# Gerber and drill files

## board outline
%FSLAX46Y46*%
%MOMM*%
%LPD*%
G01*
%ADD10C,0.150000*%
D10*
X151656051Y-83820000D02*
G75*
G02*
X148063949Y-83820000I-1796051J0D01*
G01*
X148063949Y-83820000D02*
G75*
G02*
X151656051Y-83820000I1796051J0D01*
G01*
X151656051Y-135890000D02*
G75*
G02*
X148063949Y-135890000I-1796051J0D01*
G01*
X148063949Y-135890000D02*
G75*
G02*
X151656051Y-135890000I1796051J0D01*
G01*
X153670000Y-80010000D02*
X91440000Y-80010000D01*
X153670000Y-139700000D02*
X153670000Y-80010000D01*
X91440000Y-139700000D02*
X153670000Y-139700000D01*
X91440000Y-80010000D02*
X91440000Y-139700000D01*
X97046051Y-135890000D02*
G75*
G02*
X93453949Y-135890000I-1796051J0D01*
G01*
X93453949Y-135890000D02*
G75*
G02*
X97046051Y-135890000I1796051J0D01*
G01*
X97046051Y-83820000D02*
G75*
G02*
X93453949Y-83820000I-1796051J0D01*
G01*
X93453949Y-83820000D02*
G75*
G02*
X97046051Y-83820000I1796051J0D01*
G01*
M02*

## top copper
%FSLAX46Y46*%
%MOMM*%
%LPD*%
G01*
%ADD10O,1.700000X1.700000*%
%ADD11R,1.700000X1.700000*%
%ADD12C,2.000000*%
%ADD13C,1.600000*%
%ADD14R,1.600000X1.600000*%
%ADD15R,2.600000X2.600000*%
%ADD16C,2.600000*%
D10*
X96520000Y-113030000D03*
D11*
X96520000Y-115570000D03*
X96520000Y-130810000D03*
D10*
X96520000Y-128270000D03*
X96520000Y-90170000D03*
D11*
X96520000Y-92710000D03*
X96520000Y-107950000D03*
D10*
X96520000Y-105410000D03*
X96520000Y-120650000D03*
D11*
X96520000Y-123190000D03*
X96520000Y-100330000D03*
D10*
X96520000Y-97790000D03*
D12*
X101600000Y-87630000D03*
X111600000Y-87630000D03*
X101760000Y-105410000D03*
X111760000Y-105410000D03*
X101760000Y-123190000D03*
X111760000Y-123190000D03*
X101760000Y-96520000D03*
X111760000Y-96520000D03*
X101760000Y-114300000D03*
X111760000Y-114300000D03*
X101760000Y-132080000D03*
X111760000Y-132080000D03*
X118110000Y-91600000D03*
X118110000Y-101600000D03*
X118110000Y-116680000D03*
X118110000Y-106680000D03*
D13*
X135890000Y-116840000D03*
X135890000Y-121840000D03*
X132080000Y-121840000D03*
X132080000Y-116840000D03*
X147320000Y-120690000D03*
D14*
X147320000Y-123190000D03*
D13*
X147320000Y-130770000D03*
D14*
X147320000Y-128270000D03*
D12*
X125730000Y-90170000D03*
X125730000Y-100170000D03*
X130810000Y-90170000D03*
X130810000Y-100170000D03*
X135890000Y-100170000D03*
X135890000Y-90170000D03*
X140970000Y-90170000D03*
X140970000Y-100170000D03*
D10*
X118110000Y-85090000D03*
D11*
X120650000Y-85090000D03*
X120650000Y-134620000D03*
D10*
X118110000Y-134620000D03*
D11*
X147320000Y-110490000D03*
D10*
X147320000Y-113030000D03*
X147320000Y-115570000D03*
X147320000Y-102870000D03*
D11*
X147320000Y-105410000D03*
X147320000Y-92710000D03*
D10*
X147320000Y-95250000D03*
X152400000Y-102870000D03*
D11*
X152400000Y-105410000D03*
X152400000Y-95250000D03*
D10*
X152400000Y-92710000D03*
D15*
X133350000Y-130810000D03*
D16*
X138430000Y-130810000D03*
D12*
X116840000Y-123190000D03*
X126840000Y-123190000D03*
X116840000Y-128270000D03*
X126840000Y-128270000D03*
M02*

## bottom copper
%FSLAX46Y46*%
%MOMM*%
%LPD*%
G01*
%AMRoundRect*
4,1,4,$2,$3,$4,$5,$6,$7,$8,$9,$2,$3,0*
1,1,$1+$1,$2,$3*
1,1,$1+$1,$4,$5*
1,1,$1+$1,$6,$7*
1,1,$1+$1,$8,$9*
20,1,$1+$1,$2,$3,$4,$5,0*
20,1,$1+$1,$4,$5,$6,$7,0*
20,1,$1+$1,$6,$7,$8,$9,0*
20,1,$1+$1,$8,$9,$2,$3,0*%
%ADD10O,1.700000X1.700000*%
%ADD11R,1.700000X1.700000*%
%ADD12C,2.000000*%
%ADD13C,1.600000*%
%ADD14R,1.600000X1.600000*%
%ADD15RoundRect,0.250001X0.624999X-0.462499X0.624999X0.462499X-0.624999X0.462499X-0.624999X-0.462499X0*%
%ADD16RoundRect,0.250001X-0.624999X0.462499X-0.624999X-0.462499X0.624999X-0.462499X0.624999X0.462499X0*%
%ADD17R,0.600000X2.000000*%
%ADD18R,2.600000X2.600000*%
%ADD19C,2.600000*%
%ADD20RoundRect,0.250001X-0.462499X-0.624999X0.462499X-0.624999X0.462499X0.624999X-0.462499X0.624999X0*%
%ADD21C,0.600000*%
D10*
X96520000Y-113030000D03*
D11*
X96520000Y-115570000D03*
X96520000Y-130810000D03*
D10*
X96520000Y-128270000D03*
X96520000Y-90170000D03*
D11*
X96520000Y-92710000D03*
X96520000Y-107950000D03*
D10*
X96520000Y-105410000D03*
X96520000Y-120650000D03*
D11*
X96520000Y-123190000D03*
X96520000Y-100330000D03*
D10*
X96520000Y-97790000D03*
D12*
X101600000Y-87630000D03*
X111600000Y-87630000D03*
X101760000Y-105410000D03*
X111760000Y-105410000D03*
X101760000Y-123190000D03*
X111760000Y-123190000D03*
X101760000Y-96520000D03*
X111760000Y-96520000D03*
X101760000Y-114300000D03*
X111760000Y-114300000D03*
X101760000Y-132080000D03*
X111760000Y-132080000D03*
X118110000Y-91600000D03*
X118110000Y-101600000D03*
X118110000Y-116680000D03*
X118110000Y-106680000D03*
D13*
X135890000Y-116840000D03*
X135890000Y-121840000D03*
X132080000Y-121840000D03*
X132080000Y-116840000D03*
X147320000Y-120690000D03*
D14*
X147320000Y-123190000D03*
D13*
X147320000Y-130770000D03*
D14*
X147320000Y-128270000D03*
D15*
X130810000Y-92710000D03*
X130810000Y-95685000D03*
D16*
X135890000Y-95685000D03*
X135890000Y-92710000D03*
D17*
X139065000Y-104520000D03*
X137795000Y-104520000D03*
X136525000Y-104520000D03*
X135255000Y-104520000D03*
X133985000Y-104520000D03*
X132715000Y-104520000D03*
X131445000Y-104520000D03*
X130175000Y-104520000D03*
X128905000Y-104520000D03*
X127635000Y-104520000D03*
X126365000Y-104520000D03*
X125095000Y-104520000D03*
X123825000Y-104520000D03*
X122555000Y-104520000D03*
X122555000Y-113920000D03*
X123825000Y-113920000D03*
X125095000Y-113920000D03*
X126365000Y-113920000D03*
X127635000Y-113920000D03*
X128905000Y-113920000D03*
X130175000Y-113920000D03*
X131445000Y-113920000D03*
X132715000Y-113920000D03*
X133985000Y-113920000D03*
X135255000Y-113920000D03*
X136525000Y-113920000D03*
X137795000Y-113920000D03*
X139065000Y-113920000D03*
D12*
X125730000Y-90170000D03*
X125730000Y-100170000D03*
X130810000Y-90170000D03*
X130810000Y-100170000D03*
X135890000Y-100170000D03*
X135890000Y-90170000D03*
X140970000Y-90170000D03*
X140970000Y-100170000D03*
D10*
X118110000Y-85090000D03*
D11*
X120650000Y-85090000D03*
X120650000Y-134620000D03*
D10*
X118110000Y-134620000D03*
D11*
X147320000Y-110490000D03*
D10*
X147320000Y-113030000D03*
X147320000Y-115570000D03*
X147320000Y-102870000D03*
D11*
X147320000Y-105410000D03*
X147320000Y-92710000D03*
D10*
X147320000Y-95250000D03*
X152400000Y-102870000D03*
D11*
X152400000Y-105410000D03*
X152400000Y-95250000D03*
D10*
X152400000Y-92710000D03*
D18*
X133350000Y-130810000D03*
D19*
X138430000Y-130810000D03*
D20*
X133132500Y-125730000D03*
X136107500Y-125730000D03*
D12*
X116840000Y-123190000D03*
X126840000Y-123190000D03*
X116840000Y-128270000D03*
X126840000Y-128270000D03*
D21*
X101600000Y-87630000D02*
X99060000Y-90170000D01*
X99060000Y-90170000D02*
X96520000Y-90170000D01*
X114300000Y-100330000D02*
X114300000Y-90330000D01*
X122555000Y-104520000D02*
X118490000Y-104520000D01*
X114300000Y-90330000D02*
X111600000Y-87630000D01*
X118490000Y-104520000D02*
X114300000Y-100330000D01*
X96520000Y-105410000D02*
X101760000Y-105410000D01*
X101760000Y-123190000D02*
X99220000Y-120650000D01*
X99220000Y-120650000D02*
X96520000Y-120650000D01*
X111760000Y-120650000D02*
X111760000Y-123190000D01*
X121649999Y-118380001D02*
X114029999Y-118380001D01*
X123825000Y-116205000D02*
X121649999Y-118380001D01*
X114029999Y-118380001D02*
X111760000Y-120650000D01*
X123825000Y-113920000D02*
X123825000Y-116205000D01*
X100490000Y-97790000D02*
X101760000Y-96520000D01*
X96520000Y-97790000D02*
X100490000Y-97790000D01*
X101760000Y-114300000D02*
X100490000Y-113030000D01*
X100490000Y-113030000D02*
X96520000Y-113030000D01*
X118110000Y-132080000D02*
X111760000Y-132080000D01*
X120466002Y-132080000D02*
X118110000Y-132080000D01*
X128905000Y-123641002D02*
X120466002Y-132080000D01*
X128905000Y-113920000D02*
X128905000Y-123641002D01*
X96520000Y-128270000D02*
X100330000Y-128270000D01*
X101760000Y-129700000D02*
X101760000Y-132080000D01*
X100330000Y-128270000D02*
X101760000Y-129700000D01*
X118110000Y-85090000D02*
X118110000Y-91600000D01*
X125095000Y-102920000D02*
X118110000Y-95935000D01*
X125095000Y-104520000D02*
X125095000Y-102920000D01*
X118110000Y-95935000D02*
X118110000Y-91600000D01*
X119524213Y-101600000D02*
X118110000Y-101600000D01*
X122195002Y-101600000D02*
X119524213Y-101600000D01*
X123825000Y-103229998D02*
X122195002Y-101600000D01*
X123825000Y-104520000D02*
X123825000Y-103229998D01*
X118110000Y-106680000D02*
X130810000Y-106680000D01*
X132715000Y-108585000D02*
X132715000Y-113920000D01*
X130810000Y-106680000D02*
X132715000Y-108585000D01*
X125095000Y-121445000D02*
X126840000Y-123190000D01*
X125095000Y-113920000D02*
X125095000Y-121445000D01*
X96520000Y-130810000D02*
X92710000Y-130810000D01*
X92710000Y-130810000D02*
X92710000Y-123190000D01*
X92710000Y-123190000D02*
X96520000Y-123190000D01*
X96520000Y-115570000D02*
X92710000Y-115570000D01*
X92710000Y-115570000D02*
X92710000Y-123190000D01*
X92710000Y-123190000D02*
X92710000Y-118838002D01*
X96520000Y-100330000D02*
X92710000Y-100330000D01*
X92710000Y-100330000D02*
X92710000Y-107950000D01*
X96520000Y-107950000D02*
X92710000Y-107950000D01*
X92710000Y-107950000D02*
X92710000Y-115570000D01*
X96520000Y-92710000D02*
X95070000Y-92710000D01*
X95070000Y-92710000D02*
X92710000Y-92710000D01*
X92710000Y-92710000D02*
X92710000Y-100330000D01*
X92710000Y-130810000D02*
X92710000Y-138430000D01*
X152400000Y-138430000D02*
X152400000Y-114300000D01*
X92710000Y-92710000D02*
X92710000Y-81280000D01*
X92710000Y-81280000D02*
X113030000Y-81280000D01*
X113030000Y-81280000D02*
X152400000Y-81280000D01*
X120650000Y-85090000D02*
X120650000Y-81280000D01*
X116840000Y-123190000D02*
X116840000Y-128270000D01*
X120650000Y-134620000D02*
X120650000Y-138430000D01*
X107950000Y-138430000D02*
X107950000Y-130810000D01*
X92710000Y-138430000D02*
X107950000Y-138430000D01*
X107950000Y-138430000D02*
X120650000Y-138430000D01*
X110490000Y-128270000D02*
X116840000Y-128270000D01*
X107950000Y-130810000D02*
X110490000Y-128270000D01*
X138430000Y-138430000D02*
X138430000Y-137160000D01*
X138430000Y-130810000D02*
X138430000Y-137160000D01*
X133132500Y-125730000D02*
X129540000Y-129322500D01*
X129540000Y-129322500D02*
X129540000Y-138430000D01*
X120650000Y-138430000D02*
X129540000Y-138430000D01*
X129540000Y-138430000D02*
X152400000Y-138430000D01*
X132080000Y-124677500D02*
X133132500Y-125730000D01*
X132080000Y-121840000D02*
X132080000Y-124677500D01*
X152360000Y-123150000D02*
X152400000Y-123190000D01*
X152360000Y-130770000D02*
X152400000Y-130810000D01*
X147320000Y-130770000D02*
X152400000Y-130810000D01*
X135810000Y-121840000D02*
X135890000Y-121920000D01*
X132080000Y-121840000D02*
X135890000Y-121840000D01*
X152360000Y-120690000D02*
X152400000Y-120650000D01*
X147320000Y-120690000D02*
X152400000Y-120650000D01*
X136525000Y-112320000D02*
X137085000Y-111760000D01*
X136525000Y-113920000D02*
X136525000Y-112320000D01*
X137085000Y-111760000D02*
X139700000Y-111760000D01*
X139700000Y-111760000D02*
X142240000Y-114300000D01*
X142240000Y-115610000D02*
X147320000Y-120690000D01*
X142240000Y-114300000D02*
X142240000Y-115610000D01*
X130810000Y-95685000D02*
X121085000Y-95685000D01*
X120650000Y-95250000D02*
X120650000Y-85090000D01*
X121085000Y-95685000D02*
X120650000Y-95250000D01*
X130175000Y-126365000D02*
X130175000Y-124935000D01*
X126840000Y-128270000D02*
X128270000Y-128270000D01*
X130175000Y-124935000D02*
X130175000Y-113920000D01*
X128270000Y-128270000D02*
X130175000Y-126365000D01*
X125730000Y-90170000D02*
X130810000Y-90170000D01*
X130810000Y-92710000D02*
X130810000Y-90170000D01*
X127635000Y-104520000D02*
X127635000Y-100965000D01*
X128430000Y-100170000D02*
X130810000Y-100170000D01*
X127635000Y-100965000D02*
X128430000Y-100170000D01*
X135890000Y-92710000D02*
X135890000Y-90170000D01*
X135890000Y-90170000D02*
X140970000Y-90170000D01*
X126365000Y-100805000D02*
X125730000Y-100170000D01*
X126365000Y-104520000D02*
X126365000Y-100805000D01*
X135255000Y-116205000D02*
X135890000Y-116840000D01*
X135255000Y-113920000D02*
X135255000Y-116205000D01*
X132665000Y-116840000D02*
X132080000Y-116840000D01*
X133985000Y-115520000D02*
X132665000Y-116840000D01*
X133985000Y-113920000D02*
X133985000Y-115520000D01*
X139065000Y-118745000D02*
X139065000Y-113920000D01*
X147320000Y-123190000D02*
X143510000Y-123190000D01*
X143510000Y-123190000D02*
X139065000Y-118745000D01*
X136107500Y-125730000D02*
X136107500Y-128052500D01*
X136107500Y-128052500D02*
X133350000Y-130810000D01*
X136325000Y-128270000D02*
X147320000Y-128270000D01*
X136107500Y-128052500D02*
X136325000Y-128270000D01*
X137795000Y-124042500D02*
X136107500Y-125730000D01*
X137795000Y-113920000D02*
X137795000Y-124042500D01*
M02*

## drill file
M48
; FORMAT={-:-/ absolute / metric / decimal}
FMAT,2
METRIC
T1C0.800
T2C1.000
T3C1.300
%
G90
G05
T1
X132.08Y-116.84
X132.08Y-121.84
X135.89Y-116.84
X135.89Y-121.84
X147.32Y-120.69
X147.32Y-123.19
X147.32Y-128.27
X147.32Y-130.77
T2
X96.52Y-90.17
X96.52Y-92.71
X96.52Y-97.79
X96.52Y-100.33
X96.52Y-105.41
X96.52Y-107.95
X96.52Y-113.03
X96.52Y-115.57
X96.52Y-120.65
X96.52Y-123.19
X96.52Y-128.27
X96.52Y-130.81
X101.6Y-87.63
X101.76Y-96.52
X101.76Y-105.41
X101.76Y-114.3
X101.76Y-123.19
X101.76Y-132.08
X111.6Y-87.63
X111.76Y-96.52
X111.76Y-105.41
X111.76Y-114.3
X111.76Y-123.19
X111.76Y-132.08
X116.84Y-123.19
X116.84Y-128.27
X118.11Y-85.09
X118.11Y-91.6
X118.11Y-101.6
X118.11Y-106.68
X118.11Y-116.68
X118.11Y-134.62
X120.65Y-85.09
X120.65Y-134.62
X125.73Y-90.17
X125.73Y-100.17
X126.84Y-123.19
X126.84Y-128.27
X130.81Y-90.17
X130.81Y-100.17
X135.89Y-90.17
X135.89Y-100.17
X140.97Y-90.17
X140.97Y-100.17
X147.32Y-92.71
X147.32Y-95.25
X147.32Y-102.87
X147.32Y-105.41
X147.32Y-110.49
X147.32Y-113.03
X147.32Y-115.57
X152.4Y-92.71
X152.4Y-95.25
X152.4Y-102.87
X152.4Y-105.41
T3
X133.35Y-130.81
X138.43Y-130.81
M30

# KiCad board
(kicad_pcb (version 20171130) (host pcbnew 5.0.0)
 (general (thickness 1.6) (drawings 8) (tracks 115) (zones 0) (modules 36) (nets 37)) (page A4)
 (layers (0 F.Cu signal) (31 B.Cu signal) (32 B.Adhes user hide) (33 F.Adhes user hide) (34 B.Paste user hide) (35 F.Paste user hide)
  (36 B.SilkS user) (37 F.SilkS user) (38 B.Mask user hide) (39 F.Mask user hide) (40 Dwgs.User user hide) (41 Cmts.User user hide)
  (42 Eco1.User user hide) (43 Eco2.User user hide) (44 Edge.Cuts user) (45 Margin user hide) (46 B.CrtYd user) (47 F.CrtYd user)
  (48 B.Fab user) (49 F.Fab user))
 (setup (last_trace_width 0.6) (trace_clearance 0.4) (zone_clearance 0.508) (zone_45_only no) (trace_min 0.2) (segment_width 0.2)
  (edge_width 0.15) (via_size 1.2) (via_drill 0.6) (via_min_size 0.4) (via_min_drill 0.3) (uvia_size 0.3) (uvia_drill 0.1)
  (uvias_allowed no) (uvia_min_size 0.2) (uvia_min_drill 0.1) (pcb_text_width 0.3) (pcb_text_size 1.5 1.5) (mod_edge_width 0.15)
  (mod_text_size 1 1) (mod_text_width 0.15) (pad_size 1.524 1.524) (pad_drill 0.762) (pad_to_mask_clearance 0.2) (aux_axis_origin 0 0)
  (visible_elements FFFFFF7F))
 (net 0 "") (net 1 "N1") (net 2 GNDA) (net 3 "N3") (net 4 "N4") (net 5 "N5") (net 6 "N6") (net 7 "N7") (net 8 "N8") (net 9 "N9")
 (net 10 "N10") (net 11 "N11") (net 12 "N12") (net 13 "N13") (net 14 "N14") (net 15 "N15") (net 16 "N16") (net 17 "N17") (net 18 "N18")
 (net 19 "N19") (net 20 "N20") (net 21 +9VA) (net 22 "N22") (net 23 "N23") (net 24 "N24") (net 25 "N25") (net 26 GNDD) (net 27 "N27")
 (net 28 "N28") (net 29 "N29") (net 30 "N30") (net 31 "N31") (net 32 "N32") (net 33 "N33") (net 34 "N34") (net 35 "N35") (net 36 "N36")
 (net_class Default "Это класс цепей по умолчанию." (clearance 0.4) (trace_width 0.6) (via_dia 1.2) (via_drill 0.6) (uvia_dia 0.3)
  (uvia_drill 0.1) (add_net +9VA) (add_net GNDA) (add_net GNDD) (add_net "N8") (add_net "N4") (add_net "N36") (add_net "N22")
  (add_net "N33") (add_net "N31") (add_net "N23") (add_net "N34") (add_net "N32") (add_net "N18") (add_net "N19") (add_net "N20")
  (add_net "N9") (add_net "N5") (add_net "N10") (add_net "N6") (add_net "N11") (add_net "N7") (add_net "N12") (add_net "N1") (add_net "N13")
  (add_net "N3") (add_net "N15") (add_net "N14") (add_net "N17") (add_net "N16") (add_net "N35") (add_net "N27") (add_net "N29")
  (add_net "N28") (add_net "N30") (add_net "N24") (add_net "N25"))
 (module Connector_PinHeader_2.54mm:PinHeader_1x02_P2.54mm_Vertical (layer F.Cu) (at 96.52 115.57 180)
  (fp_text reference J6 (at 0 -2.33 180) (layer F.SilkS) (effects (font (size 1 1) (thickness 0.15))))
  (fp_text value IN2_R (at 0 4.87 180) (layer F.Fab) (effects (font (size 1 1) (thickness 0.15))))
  (pad 2 thru_hole oval (at 0 2.54 180) (size 1.7 1.7) (drill 1) (layers *.Cu *.Mask) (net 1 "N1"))
  (pad 1 thru_hole rect (at 0 0 180) (size 1.7 1.7) (drill 1) (layers *.Cu *.Mask) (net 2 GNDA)))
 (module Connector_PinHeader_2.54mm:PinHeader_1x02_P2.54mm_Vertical (layer F.Cu) (at 96.52 130.81 180)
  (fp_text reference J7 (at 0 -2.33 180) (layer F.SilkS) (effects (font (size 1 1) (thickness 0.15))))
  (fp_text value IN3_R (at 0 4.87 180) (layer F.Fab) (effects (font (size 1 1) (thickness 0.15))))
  (pad 1 thru_hole rect (at 0 0 180) (size 1.7 1.7) (drill 1) (layers *.Cu *.Mask) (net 2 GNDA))
  (pad 2 thru_hole oval (at 0 2.54 180) (size 1.7 1.7) (drill 1) (layers *.Cu *.Mask) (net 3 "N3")))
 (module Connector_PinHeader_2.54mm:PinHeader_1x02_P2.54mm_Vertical (layer F.Cu) (at 96.52 92.71 180)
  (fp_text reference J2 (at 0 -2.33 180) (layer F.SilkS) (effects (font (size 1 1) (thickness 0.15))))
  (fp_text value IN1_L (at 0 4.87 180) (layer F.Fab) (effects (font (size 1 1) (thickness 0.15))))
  (pad 2 thru_hole oval (at 0 2.54 180) (size 1.7 1.7) (drill 1) (layers *.Cu *.Mask) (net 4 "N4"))
  (pad 1 thru_hole rect (at 0 0 180) (size 1.7 1.7) (drill 1) (layers *.Cu *.Mask) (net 2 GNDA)))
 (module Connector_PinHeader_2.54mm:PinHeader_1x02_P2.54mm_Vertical (layer F.Cu) (at 96.52 107.95 180)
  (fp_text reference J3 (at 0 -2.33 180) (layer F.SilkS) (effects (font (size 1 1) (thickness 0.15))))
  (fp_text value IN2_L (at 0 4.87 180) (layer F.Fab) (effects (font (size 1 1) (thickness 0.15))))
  (pad 1 thru_hole rect (at 0 0 180) (size 1.7 1.7) (drill 1) (layers *.Cu *.Mask) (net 2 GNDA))
  (pad 2 thru_hole oval (at 0 2.54 180) (size 1.7 1.7) (drill 1) (layers *.Cu *.Mask) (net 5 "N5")))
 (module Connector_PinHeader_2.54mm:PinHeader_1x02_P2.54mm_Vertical (layer F.Cu) (at 96.52 123.19 180)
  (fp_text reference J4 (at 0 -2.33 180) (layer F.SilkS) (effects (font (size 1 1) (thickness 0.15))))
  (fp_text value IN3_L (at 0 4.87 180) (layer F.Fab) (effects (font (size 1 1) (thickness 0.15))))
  (pad 2 thru_hole oval (at 0 2.54 180) (size 1.7 1.7) (drill 1) (layers *.Cu *.Mask) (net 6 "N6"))
  (pad 1 thru_hole rect (at 0 0 180) (size 1.7 1.7) (drill 1) (layers *.Cu *.Mask) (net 2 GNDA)))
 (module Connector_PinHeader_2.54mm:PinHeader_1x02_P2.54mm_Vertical (layer F.Cu) (at 96.52 100.33 180)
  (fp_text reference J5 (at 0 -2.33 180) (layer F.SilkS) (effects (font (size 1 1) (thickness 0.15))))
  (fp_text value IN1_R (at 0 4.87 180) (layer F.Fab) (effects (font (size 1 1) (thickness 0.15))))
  (pad 1 thru_hole rect (at 0 0 180) (size 1.7 1.7) (drill 1) (layers *.Cu *.Mask) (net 2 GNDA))
  (pad 2 thru_hole oval (at 0 2.54 180) (size 1.7 1.7) (drill 1) (layers *.Cu *.Mask) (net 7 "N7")))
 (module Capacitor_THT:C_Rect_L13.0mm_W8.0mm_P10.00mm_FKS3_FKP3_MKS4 (layer F.Cu) (at 111.6 87.63 180)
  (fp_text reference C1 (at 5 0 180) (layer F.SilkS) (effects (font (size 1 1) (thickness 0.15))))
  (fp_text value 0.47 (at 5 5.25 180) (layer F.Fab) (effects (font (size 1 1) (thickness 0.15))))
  (pad 2 thru_hole circle (at 10 0 180) (size 2 2) (drill 1) (layers *.Cu *.Mask) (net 4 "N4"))
  (pad 1 thru_hole circle (at 0 0 180) (size 2 2) (drill 1) (layers *.Cu *.Mask) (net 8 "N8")))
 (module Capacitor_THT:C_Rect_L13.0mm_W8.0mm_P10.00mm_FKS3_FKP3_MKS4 (layer F.Cu) (at 111.76 105.41 180)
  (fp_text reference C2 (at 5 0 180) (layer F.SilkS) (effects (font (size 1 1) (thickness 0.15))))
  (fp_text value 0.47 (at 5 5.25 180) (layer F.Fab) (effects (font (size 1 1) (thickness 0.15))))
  (pad 2 thru_hole circle (at 10 0 180) (size 2 2) (drill 1) (layers *.Cu *.Mask) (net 5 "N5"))
  (pad 1 thru_hole circle (at 0 0 180) (size 2 2) (drill 1) (layers *.Cu *.Mask) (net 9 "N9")))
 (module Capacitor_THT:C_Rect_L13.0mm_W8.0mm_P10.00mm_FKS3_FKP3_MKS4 (layer F.Cu) (at 111.76 123.19 180)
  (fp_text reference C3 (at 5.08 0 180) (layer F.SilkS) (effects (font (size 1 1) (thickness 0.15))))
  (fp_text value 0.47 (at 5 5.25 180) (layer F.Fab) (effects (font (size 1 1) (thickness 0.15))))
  (pad 2 thru_hole circle (at 10 0 180) (size 2 2) (drill 1) (layers *.Cu *.Mask) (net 6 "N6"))
  (pad 1 thru_hole circle (at 0 0 180) (size 2 2) (drill 1) (layers *.Cu *.Mask) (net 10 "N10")))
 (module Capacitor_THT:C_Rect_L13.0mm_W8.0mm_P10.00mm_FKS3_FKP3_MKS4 (layer F.Cu) (at 111.76 96.52 180)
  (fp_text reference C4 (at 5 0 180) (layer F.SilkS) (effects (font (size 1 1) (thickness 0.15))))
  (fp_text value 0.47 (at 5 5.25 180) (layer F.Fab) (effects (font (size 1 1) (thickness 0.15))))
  (pad 2 thru_hole circle (at 10 0 180) (size 2 2) (drill 1) (layers *.Cu *.Mask) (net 7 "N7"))
  (pad 1 thru_hole circle (at 0 0 180) (size 2 2) (drill 1) (layers *.Cu *.Mask) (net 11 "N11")))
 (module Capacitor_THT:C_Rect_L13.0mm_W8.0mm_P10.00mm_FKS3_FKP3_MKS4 (layer F.Cu) (at 111.76 114.3 180)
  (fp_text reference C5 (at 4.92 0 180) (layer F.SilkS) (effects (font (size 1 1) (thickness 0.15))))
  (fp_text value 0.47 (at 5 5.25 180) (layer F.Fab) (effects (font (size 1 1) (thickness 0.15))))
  (pad 2 thru_hole circle (at 10 0 180) (size 2 2) (drill 1) (layers *.Cu *.Mask) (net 1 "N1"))
  (pad 1 thru_hole circle (at 0 0 180) (size 2 2) (drill 1) (layers *.Cu *.Mask) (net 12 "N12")))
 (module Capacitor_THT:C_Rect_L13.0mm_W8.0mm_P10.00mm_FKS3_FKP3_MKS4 (layer F.Cu) (at 111.76 132.08 180)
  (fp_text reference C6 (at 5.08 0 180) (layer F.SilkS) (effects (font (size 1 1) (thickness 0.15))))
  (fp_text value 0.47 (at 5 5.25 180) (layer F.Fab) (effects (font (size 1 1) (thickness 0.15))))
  (pad 2 thru_hole circle (at 10 0 180) (size 2 2) (drill 1) (layers *.Cu *.Mask) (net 3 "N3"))
  (pad 1 thru_hole circle (at 0 0 180) (size 2 2) (drill 1) (layers *.Cu *.Mask) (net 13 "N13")))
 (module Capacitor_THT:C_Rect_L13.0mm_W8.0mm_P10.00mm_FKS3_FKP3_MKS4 (layer F.Cu) (at 118.11 101.6 90)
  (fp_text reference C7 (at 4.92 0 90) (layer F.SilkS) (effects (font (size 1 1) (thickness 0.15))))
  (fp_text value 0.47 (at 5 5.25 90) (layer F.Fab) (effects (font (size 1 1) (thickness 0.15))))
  (pad 2 thru_hole circle (at 10 0 90) (size 2 2) (drill 1) (layers *.Cu *.Mask) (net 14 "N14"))
  (pad 1 thru_hole circle (at 0 0 90) (size 2 2) (drill 1) (layers *.Cu *.Mask) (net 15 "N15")))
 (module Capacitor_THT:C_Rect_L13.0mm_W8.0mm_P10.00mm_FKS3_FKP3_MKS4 (layer F.Cu) (at 118.11 106.68 270)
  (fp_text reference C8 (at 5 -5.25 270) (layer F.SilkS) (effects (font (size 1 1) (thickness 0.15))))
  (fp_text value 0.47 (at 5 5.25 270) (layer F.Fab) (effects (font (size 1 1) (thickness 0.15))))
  (pad 2 thru_hole circle (at 10 0 270) (size 2 2) (drill 1) (layers *.Cu *.Mask) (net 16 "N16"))
  (pad 1 thru_hole circle (at 0 0 270) (size 2 2) (drill 1) (layers *.Cu *.Mask) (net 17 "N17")))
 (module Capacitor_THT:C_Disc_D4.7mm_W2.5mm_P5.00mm (layer F.Cu) (at 135.89 121.84 90)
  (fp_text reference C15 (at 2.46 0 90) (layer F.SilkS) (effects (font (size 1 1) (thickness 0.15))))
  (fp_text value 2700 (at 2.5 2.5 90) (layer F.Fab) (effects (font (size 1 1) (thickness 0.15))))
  (pad 2 thru_hole circle (at 5 0 90) (size 1.6 1.6) (drill 0.8) (layers *.Cu *.Mask) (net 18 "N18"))
  (pad 1 thru_hole circle (at 0 0 90) (size 1.6 1.6) (drill 0.8) (layers *.Cu *.Mask) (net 2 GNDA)))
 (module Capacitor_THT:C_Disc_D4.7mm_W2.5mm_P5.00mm (layer F.Cu) (at 132.08 116.84 270)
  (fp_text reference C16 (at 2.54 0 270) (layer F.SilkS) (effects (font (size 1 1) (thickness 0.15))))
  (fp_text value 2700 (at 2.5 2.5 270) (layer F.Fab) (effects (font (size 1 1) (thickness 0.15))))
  (pad 2 thru_hole circle (at 5 0 270) (size 1.6 1.6) (drill 0.8) (layers *.Cu *.Mask) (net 2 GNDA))
  (pad 1 thru_hole circle (at 0 0 270) (size 1.6 1.6) (drill 0.8) (layers *.Cu *.Mask) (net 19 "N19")))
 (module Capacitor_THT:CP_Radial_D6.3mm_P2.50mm (layer F.Cu) (at 147.32 123.19 90)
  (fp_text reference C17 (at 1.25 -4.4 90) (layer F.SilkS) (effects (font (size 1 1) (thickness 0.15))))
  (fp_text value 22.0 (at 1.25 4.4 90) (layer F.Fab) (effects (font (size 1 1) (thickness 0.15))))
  (pad 2 thru_hole circle (at 2.5 0 90) (size 1.6 1.6) (drill 0.8) (layers *.Cu *.Mask) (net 2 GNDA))
  (pad 1 thru_hole rect (at 0 0 90) (size 1.6 1.6) (drill 0.8) (layers *.Cu *.Mask) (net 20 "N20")))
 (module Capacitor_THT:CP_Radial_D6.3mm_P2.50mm (layer F.Cu) (at 147.32 128.27 270)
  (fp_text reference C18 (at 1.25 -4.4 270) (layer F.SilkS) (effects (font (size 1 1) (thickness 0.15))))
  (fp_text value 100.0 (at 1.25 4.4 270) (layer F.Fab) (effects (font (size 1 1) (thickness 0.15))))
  (pad 2 thru_hole circle (at 2.5 0 270) (size 1.6 1.6) (drill 0.8) (layers *.Cu *.Mask) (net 2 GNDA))
  (pad 1 thru_hole rect (at 0 0 270) (size 1.6 1.6) (drill 0.8) (layers *.Cu *.Mask) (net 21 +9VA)))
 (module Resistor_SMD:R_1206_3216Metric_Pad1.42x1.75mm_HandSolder (layer B.Cu) (at 130.81 94.1975 90)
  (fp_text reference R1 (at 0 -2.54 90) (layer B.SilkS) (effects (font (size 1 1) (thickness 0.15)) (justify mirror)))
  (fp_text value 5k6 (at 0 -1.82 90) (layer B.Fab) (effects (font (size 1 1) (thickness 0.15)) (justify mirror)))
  (pad 2 smd roundrect (at 1.4875 0 90) (size 1.425 1.75) (layers B.Cu B.Paste B.Mask) (roundrect_rratio 0.175439) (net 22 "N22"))
  (pad 1 smd roundrect (at -1.4875 0 90) (size 1.425 1.75) (layers B.Cu B.Paste B.Mask) (roundrect_rratio 0.175439) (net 2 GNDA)))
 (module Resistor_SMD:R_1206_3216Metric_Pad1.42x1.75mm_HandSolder (layer B.Cu) (at 135.89 94.1975 270)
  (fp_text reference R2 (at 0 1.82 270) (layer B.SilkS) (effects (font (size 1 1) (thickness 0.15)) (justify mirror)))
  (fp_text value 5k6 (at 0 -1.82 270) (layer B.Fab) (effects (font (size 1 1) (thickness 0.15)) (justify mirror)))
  (pad 2 smd roundrect (at 1.4875 0 270) (size 1.425 1.75) (layers B.Cu B.Paste B.Mask) (roundrect_rratio 0.175439) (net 2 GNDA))
  (pad 1 smd roundrect (at -1.4875 0 270) (size 1.425 1.75) (layers B.Cu B.Paste B.Mask) (roundrect_rratio 0.175439) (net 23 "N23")))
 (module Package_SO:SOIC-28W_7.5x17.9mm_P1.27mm (layer B.Cu) (at 130.81 109.22 90)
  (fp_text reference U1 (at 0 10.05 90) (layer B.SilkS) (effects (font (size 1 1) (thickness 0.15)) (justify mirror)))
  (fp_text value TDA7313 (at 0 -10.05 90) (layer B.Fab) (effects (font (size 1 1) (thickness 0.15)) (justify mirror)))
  (pad 28 smd rect (at 4.7 8.255 90) (size 2 0.6) (layers B.Cu B.Paste B.Mask) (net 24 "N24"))
  (pad 27 smd rect (at 4.7 6.985 90) (size 2 0.6) (layers B.Cu B.Paste B.Mask) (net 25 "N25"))
  (pad 26 smd rect (at 4.7 5.715 90) (size 2 0.6) (layers B.Cu B.Paste B.Mask) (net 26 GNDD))
  (pad 25 smd rect (at 4.7 4.445 90) (size 2 0.6) (layers B.Cu B.Paste B.Mask) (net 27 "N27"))
  (pad 24 smd rect (at 4.7 3.175 90) (size 2 0.6) (layers B.Cu B.Paste B.Mask) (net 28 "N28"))
  (pad 23 smd rect (at 4.7 1.905 90) (size 2 0.6) (layers B.Cu B.Paste B.Mask) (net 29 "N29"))
  (pad 22 smd rect (at 4.7 0.635 90) (size 2 0.6) (layers B.Cu B.Paste B.Mask) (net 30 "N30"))
  (pad 21 smd rect (at 4.7 -0.635 90) (size 2 0.6) (layers B.Cu B.Paste B.Mask) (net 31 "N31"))
  (pad 20 smd rect (at 4.7 -1.905 90) (size 2 0.6) (layers B.Cu B.Paste B.Mask) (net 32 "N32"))
  (pad 19 smd rect (at 4.7 -3.175 90) (size 2 0.6) (layers B.Cu B.Paste B.Mask) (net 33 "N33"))
  (pad 18 smd rect (at 4.7 -4.445 90) (size 2 0.6) (layers B.Cu B.Paste B.Mask) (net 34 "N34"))
  (pad 17 smd rect (at 4.7 -5.715 90) (size 2 0.6) (layers B.Cu B.Paste B.Mask) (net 14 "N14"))
  (pad 16 smd rect (at 4.7 -6.985 90) (size 2 0.6) (layers B.Cu B.Paste B.Mask) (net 15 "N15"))
  (pad 15 smd rect (at 4.7 -8.255 90) (size 2 0.6) (layers B.Cu B.Paste B.Mask) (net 8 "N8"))
  (pad 14 smd rect (at -4.7 -8.255 90) (size 2 0.6) (layers B.Cu B.Paste B.Mask) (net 9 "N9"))
  (pad 13 smd rect (at -4.7 -6.985 90) (size 2 0.6) (layers B.Cu B.Paste B.Mask) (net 10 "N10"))
  (pad 12 smd rect (at -4.7 -5.715 90) (size 2 0.6) (layers B.Cu B.Paste B.Mask) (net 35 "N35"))
  (pad 11 smd rect (at -4.7 -4.445 90) (size 2 0.6) (layers B.Cu B.Paste B.Mask) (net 11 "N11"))
  (pad 10 smd rect (at -4.7 -3.175 90) (size 2 0.6) (layers B.Cu B.Paste B.Mask) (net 12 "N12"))
  (pad 9 smd rect (at -4.7 -1.905 90) (size 2 0.6) (layers B.Cu B.Paste B.Mask) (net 13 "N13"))
  (pad 8 smd rect (at -4.7 -0.635 90) (size 2 0.6) (layers B.Cu B.Paste B.Mask) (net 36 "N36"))
  (pad 7 smd rect (at -4.7 0.635 90) (size 2 0.6) (layers B.Cu B.Paste B.Mask) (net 16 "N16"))
  (pad 6 smd rect (at -4.7 1.905 90) (size 2 0.6) (layers B.Cu B.Paste B.Mask) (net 17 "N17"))
  (pad 5 smd rect (at -4.7 3.175 90) (size 2 0.6) (layers B.Cu B.Paste B.Mask) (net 19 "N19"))
  (pad 4 smd rect (at -4.7 4.445 90) (size 2 0.6) (layers B.Cu B.Paste B.Mask) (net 18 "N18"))
  (pad 3 smd rect (at -4.7 5.715 90) (size 2 0.6) (layers B.Cu B.Paste B.Mask) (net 2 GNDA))
  (pad 2 smd rect (at -4.7 6.985 90) (size 2 0.6) (layers B.Cu B.Paste B.Mask) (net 21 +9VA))
  (pad 1 smd rect (at -4.7 8.255 90) (size 2 0.6) (layers B.Cu B.Paste B.Mask) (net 20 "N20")))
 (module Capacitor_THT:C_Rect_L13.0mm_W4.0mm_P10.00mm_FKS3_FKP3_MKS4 (layer F.Cu) (at 125.73 90.17 270)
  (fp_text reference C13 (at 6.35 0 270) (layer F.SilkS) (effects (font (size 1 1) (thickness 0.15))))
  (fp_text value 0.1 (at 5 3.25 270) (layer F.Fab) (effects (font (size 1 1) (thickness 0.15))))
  (pad 1 thru_hole circle (at 0 0 270) (size 2 2) (drill 1) (layers *.Cu *.Mask) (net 22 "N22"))
  (pad 2 thru_hole circle (at 10 0 270) (size 2 2) (drill 1) (layers *.Cu *.Mask) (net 34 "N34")))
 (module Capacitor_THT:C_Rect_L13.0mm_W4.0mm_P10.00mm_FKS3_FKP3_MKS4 (layer F.Cu) (at 130.81 90.17 270)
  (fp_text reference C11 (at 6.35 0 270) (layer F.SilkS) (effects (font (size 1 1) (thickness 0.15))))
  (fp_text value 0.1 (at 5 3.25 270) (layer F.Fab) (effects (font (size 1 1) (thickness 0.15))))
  (pad 1 thru_hole circle (at 0 0 270) (size 2 2) (drill 1) (layers *.Cu *.Mask) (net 22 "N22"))
  (pad 2 thru_hole circle (at 10 0 270) (size 2 2) (drill 1) (layers *.Cu *.Mask) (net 33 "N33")))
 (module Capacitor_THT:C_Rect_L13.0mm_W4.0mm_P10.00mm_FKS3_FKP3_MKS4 (layer F.Cu) (at 135.89 100.17 90)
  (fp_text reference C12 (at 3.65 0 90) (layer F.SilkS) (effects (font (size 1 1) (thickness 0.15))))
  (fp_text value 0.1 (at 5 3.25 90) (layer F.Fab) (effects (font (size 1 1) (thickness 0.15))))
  (pad 1 thru_hole circle (at 0 0 90) (size 2 2) (drill 1) (layers *.Cu *.Mask) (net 31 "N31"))
  (pad 2 thru_hole circle (at 10 0 90) (size 2 2) (drill 1) (layers *.Cu *.Mask) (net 23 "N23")))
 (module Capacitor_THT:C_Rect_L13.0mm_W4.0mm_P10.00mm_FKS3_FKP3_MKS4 (layer F.Cu) (at 140.97 100.17 90)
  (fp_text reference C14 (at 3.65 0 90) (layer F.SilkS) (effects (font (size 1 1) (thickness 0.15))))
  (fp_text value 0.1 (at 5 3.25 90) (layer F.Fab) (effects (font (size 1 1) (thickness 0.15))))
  (pad 2 thru_hole circle (at 10 0 90) (size 2 2) (drill 1) (layers *.Cu *.Mask) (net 23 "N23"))
  (pad 1 thru_hole circle (at 0 0 90) (size 2 2) (drill 1) (layers *.Cu *.Mask) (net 32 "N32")))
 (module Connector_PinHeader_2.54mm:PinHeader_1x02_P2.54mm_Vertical (layer F.Cu) (at 120.65 85.09 270)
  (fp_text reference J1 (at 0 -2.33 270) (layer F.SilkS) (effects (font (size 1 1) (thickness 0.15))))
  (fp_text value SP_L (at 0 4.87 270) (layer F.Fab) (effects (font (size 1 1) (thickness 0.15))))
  (pad 2 thru_hole oval (at 0 2.54 270) (size 1.7 1.7) (drill 1) (layers *.Cu *.Mask) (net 14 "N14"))
  (pad 1 thru_hole rect (at 0 0 270) (size 1.7 1.7) (drill 1) (layers *.Cu *.Mask) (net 2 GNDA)))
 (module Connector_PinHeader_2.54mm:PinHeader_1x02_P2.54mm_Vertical (layer F.Cu) (at 120.65 134.62 270)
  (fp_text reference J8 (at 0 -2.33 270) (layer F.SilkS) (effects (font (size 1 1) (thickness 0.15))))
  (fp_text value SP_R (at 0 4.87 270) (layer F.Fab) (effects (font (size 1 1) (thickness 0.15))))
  (pad 1 thru_hole rect (at 0 0 270) (size 1.7 1.7) (drill 1) (layers *.Cu *.Mask) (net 2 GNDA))
  (pad 2 thru_hole oval (at 0 2.54 270) (size 1.7 1.7) (drill 1) (layers *.Cu *.Mask) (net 16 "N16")))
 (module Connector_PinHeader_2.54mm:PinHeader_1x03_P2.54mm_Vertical (layer F.Cu) (at 147.32 110.49)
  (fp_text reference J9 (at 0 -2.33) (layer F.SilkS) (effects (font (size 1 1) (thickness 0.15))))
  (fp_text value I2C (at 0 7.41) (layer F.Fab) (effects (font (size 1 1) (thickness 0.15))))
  (pad 1 thru_hole rect (at 0 0) (size 1.7 1.7) (drill 1) (layers *.Cu *.Mask) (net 24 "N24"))
  (pad 2 thru_hole oval (at 0 2.54) (size 1.7 1.7) (drill 1) (layers *.Cu *.Mask) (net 25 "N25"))
  (pad 3 thru_hole oval (at 0 5.08) (size 1.7 1.7) (drill 1) (layers *.Cu *.Mask) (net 26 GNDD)))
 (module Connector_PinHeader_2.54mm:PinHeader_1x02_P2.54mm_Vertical (layer F.Cu) (at 147.32 105.41 180)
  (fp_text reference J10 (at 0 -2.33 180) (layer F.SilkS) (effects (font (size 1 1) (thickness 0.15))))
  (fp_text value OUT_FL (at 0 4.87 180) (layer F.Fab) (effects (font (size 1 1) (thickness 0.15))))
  (pad 2 thru_hole oval (at 0 2.54 180) (size 1.7 1.7) (drill 1) (layers *.Cu *.Mask) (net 27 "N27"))
  (pad 1 thru_hole rect (at 0 0 180) (size 1.7 1.7) (drill 1) (layers *.Cu *.Mask) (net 2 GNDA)))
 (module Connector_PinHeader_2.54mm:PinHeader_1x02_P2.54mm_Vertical (layer F.Cu) (at 147.32 92.71)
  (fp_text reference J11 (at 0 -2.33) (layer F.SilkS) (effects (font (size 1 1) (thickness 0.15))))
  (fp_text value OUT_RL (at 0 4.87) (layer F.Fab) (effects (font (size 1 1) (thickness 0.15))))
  (pad 1 thru_hole rect (at 0 0) (size 1.7 1.7) (drill 1) (layers *.Cu *.Mask) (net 2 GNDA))
  (pad 2 thru_hole oval (at 0 2.54) (size 1.7 1.7) (drill 1) (layers *.Cu *.Mask) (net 29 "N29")))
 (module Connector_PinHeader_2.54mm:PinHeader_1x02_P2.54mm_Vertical (layer F.Cu) (at 152.4 105.41 180)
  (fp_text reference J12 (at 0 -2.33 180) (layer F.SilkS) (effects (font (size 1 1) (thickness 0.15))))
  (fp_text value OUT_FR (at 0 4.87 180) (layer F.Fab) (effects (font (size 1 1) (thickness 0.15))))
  (pad 2 thru_hole oval (at 0 2.54 180) (size 1.7 1.7) (drill 1) (layers *.Cu *.Mask) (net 28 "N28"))
  (pad 1 thru_hole rect (at 0 0 180) (size 1.7 1.7) (drill 1) (layers *.Cu *.Mask) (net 2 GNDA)))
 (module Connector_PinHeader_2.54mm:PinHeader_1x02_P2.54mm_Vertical (layer F.Cu) (at 152.4 95.25 180)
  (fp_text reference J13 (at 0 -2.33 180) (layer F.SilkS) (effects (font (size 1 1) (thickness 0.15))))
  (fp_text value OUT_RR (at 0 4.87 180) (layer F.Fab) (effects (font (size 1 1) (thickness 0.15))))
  (pad 1 thru_hole rect (at 0 0 180) (size 1.7 1.7) (drill 1) (layers *.Cu *.Mask) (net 2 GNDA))
  (pad 2 thru_hole oval (at 0 2.54 180) (size 1.7 1.7) (drill 1) (layers *.Cu *.Mask) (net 30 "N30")))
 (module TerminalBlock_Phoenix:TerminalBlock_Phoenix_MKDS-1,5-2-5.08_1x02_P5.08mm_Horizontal (layer F.Cu) (at 133.35 130.81)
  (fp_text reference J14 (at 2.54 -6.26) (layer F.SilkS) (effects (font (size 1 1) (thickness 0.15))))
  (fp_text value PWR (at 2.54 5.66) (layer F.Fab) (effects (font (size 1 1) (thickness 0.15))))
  (pad 1 thru_hole rect (at 0 0) (size 2.6 2.6) (drill 1.3) (layers *.Cu *.Mask) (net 21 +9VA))
  (pad 2 thru_hole circle (at 5.08 0) (size 2.6 2.6) (drill 1.3) (layers *.Cu *.Mask) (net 2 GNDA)))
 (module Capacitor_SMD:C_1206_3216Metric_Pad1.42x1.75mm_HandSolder (layer B.Cu) (at 134.62 125.73)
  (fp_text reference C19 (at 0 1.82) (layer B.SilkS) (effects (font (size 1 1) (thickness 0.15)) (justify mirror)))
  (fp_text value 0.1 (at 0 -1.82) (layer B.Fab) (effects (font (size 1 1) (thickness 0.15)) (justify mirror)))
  (pad 1 smd roundrect (at -1.4875 0) (size 1.425 1.75) (layers B.Cu B.Paste B.Mask) (roundrect_rratio 0.175439) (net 2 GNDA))
  (pad 2 smd roundrect (at 1.4875 0) (size 1.425 1.75) (layers B.Cu B.Paste B.Mask) (roundrect_rratio 0.175439) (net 21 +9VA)))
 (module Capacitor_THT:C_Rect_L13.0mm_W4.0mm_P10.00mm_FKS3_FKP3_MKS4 (layer F.Cu) (at 116.84 123.19)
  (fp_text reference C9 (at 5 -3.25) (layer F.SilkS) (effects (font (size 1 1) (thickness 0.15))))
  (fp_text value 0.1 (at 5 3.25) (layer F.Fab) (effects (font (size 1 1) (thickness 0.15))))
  (pad 1 thru_hole circle (at 0 0) (size 2 2) (drill 1) (layers *.Cu *.Mask) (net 2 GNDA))
  (pad 2 thru_hole circle (at 10 0) (size 2 2) (drill 1) (layers *.Cu *.Mask) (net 35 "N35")))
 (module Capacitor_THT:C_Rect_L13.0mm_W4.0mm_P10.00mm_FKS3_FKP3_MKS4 (layer F.Cu) (at 126.84 128.27 180)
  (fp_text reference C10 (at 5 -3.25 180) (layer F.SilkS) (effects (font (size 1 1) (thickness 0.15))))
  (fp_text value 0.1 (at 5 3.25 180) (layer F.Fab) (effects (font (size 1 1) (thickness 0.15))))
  (pad 2 thru_hole circle (at 10 0 180) (size 2 2) (drill 1) (layers *.Cu *.Mask) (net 2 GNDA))
  (pad 1 thru_hole circle (at 0 0 180) (size 2 2) (drill 1) (layers *.Cu *.Mask) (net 36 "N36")))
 (gr_circle (center 149.86 83.82) (end 151.13 82.55) (layer Edge.Cuts) (width 0.15))
 (gr_circle (center 149.86 135.89) (end 151.13 134.62) (layer Edge.Cuts) (width 0.15))
 (gr_line (start 153.67 80.01) (end 91.44 80.01) (layer Edge.Cuts) (width 0.15))
 (gr_line (start 153.67 139.7) (end 153.67 80.01) (layer Edge.Cuts) (width 0.15))
 (gr_line (start 91.44 139.7) (end 153.67 139.7) (layer Edge.Cuts) (width 0.15))
 (gr_line (start 91.44 80.01) (end 91.44 139.7) (layer Edge.Cuts) (width 0.15))
 (gr_circle (center 95.25 135.89) (end 96.52 137.16) (layer Edge.Cuts) (width 0.15))
 (gr_circle (center 95.25 83.82) (end 96.52 82.55) (layer Edge.Cuts) (width 0.15))
 (segment (start 101.6 87.63) (end 99.06 90.17) (width 0.6) (layer B.Cu) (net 4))
 (segment (start 99.06 90.17) (end 96.52 90.17) (width 0.6) (layer B.Cu) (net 4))
 (segment (start 114.3 100.33) (end 114.3 90.33) (width 0.6) (layer B.Cu) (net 8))
 (segment (start 122.555 104.52) (end 118.49 104.52) (width 0.6) (layer B.Cu) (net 8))
 (segment (start 114.3 90.33) (end 111.6 87.63) (width 0.6) (layer B.Cu) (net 8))
 (segment (start 118.49 104.52) (end 114.3 100.33) (width 0.6) (layer B.Cu) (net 8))
 (segment (start 96.52 105.41) (end 101.76 105.41) (width 0.6) (layer B.Cu) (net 5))
 (segment (start 101.76 123.19) (end 99.22 120.65) (width 0.6) (layer B.Cu) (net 6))
 (segment (start 99.22 120.65) (end 96.52 120.65) (width 0.6) (layer B.Cu) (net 6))
 (segment (start 111.76 120.65) (end 111.76 123.19) (width 0.6) (layer B.Cu) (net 10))
 (segment (start 121.649999 118.380001) (end 114.029999 118.380001) (width 0.6) (layer B.Cu) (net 10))
 (segment (start 123.825 116.205) (end 121.649999 118.380001) (width 0.6) (layer B.Cu) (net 10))
 (segment (start 114.029999 118.380001) (end 111.76 120.65) (width 0.6) (layer B.Cu) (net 10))
 (segment (start 123.825 113.92) (end 123.825 116.205) (width 0.6) (layer B.Cu) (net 10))
 (segment (start 100.49 97.79) (end 101.76 96.52) (width 0.6) (layer B.Cu) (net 7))
 (segment (start 96.52 97.79) (end 100.49 97.79) (width 0.6) (layer B.Cu) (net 7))
 (segment (start 101.76 114.3) (end 100.49 113.03) (width 0.6) (layer B.Cu) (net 1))
 (segment (start 100.49 113.03) (end 96.52 113.03) (width 0.6) (layer B.Cu) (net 1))
 (segment (start 118.11 132.08) (end 111.76 132.08) (width 0.6) (layer B.Cu) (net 13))
 (segment (start 120.466002 132.08) (end 118.11 132.08) (width 0.6) (layer B.Cu) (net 13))
 (segment (start 128.905 123.641002) (end 120.466002 132.08) (width 0.6) (layer B.Cu) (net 13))
 (segment (start 128.905 113.92) (end 128.905 123.641002) (width 0.6) (layer B.Cu) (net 13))
 (segment (start 96.52 128.27) (end 100.33 128.27) (width 0.6) (layer B.Cu) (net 3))
 (segment (start 101.76 129.7) (end 101.76 132.08) (width 0.6) (layer B.Cu) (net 3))
 (segment (start 100.33 128.27) (end 101.76 129.7) (width 0.6) (layer B.Cu) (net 3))
 (segment (start 118.11 85.09) (end 118.11 91.6) (width 0.6) (layer B.Cu) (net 14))
 (segment (start 125.095 102.92) (end 118.11 95.935) (width 0.6) (layer B.Cu) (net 14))
 (segment (start 125.095 104.52) (end 125.095 102.92) (width 0.6) (layer B.Cu) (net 14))
 (segment (start 118.11 95.935) (end 118.11 91.6) (width 0.6) (layer B.Cu) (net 14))
 (segment (start 119.524213 101.6) (end 118.11 101.6) (width 0.6) (layer B.Cu) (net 15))
 (segment (start 122.195002 101.6) (end 119.524213 101.6) (width 0.6) (layer B.Cu) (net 15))
 (segment (start 123.825 103.229998) (end 122.195002 101.6) (width 0.6) (layer B.Cu) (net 15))
 (segment (start 123.825 104.52) (end 123.825 103.229998) (width 0.6) (layer B.Cu) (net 15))
 (segment (start 118.11 106.68) (end 130.81 106.68) (width 0.6) (layer B.Cu) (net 17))
 (segment (start 132.715 108.585) (end 132.715 113.92) (width 0.6) (layer B.Cu) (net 17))
 (segment (start 130.81 106.68) (end 132.715 108.585) (width 0.6) (layer B.Cu) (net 17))
 (segment (start 125.095 121.445) (end 126.84 123.19) (width 0.6) (layer B.Cu) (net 35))
 (segment (start 125.095 113.92) (end 125.095 121.445) (width 0.6) (layer B.Cu) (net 35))
 (segment (start 96.52 130.81) (end 92.71 130.81) (width 0.6) (layer B.Cu) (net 2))
 (segment (start 92.71 130.81) (end 92.71 123.19) (width 0.6) (layer B.Cu) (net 2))
 (segment (start 92.71 123.19) (end 96.52 123.19) (width 0.6) (layer B.Cu) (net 2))
 (segment (start 96.52 115.57) (end 92.71 115.57) (width 0.6) (layer B.Cu) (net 2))
 (segment (start 92.71 115.57) (end 92.71 123.19) (width 0.6) (layer B.Cu) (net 2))
 (segment (start 92.71 123.19) (end 92.71 118.838002) (width 0.6) (layer B.Cu) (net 2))
 (segment (start 96.52 100.33) (end 92.71 100.33) (width 0.6) (layer B.Cu) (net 2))
 (segment (start 92.71 100.33) (end 92.71 107.95) (width 0.6) (layer B.Cu) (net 2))
 (segment (start 96.52 107.95) (end 92.71 107.95) (width 0.6) (layer B.Cu) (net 2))
 (segment (start 92.71 107.95) (end 92.71 115.57) (width 0.6) (layer B.Cu) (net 2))
 (segment (start 96.52 92.71) (end 95.07 92.71) (width 0.6) (layer B.Cu) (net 2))
 (segment (start 95.07 92.71) (end 92.71 92.71) (width 0.6) (layer B.Cu) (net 2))
 (segment (start 92.71 92.71) (end 92.71 100.33) (width 0.6) (layer B.Cu) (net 2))
 (segment (start 92.71 130.81) (end 92.71 138.43) (width 0.6) (layer B.Cu) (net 2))
 (segment (start 152.4 138.43) (end 152.4 114.3) (width 0.6) (layer B.Cu) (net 2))
 (segment (start 92.71 92.71) (end 92.71 81.28) (width 0.6) (layer B.Cu) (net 2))
 (segment (start 92.71 81.28) (end 113.03 81.28) (width 0.6) (layer B.Cu) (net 2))
 (segment (start 113.03 81.28) (end 152.4 81.28) (width 0.6) (layer B.Cu) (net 2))
 (segment (start 120.65 85.09) (end 120.65 81.28) (width 0.6) (layer B.Cu) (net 2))
 (segment (start 116.84 123.19) (end 116.84 128.27) (width 0.6) (layer B.Cu) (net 2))
 (segment (start 120.65 134.62) (end 120.65 138.43) (width 0.6) (layer B.Cu) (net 2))
 (segment (start 107.95 138.43) (end 107.95 130.81) (width 0.6) (layer B.Cu) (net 2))
 (segment (start 92.71 138.43) (end 107.95 138.43) (width 0.6) (layer B.Cu) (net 2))
 (segment (start 107.95 138.43) (end 120.65 138.43) (width 0.6) (layer B.Cu) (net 2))
 (segment (start 110.49 128.27) (end 116.84 128.27) (width 0.6) (layer B.Cu) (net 2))
 (segment (start 107.95 130.81) (end 110.49 128.27) (width 0.6) (layer B.Cu) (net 2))
 (segment (start 138.43 138.43) (end 138.43 137.16) (width 0.6) (layer B.Cu) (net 2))
 (segment (start 138.43 130.81) (end 138.43 137.16) (width 0.6) (layer B.Cu) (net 2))
 (segment (start 133.1325 125.73) (end 129.54 129.3225) (width 0.6) (layer B.Cu) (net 2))
 (segment (start 129.54 129.3225) (end 129.54 138.43) (width 0.6) (layer B.Cu) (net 2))
 (segment (start 120.65 138.43) (end 129.54 138.43) (width 0.6) (layer B.Cu) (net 2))
 (segment (start 129.54 138.43) (end 152.4 138.43) (width 0.6) (layer B.Cu) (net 2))
 (segment (start 132.08 124.6775) (end 133.1325 125.73) (width 0.6) (layer B.Cu) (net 2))
 (segment (start 132.08 121.84) (end 132.08 124.6775) (width 0.6) (layer B.Cu) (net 2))
 (segment (start 152.36 123.15) (end 152.4 123.19) (width 0.6) (layer B.Cu) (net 2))
 (segment (start 152.36 130.77) (end 152.4 130.81) (width 0.6) (layer B.Cu) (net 2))
 (segment (start 147.32 130.77) (end 152.4 130.81) (width 0.6) (layer B.Cu) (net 2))
 (segment (start 135.81 121.84) (end 135.89 121.92) (width 0.6) (layer B.Cu) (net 2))
 (segment (start 132.08 121.84) (end 135.89 121.84) (width 0.6) (layer B.Cu) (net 2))
 (segment (start 152.36 120.69) (end 152.4 120.65) (width 0.6) (layer B.Cu) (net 2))
 (segment (start 147.32 120.69) (end 152.4 120.65) (width 0.6) (layer B.Cu) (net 2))
 (segment (start 136.525 112.32) (end 137.085 111.76) (width 0.6) (layer B.Cu) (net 2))
 (segment (start 136.525 113.92) (end 136.525 112.32) (width 0.6) (layer B.Cu) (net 2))
 (segment (start 137.085 111.76) (end 139.7 111.76) (width 0.6) (layer B.Cu) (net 2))
 (segment (start 139.7 111.76) (end 142.24 114.3) (width 0.6) (layer B.Cu) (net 2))
 (segment (start 142.24 115.61) (end 147.32 120.69) (width 0.6) (layer B.Cu) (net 2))
 (segment (start 142.24 114.3) (end 142.24 115.61) (width 0.6) (layer B.Cu) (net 2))
 (segment (start 130.81 95.685) (end 121.085 95.685) (width 0.6) (layer B.Cu) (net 2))
 (segment (start 120.65 95.25) (end 120.65 85.09) (width 0.6) (layer B.Cu) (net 2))
 (segment (start 121.085 95.685) (end 120.65 95.25) (width 0.6) (layer B.Cu) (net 2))
 (segment (start 130.175 126.365) (end 130.175 124.935) (width 0.6) (layer B.Cu) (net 36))
 (segment (start 126.84 128.27) (end 128.27 128.27) (width 0.6) (layer B.Cu) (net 36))
 (segment (start 130.175 124.935) (end 130.175 113.92) (width 0.6) (layer B.Cu) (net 36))
 (segment (start 128.27 128.27) (end 130.175 126.365) (width 0.6) (layer B.Cu) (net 36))
 (segment (start 125.73 90.17) (end 130.81 90.17) (width 0.6) (layer B.Cu) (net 22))
 (segment (start 130.81 92.71) (end 130.81 90.17) (width 0.6) (layer B.Cu) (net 22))
 (segment (start 127.635 104.52) (end 127.635 100.965) (width 0.6) (layer B.Cu) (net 33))
 (segment (start 128.43 100.17) (end 130.81 100.17) (width 0.6) (layer B.Cu) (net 33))
 (segment (start 127.635 100.965) (end 128.43 100.17) (width 0.6) (layer B.Cu) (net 33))
 (segment (start 135.89 92.71) (end 135.89 90.17) (width 0.6) (layer B.Cu) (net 23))
 (segment (start 135.89 90.17) (end 140.97 90.17) (width 0.6) (layer B.Cu) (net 23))
 (segment (start 126.365 100.805) (end 125.73 100.17) (width 0.6) (layer B.Cu) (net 34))
 (segment (start 126.365 104.52) (end 126.365 100.805) (width 0.6) (layer B.Cu) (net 34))
 (segment (start 135.255 116.205) (end 135.89 116.84) (width 0.6) (layer B.Cu) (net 18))
 (segment (start 135.255 113.92) (end 135.255 116.205) (width 0.6) (layer B.Cu) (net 18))
 (segment (start 132.665 116.84) (end 132.08 116.84) (width 0.6) (layer B.Cu) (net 19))
 (segment (start 133.985 115.52) (end 132.665 116.84) (width 0.6) (layer B.Cu) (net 19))
 (segment (start 133.985 113.92) (end 133.985 115.52) (width 0.6) (layer B.Cu) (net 19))
 (segment (start 139.065 118.745) (end 139.065 113.92) (width 0.6) (layer B.Cu) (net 20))
 (segment (start 147.32 123.19) (end 143.51 123.19) (width 0.6) (layer B.Cu) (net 20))
 (segment (start 143.51 123.19) (end 139.065 118.745) (width 0.6) (layer B.Cu) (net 20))
 (segment (start 136.1075 125.73) (end 136.1075 128.0525) (width 0.6) (layer B.Cu) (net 21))
 (segment (start 136.1075 128.0525) (end 133.35 130.81) (width 0.6) (layer B.Cu) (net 21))
 (segment (start 136.325 128.27) (end 147.32 128.27) (width 0.6) (layer B.Cu) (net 21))
 (segment (start 136.1075 128.0525) (end 136.325 128.27) (width 0.6) (layer B.Cu) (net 21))
 (segment (start 137.795 124.0425) (end 136.1075 125.73) (width 0.6) (layer B.Cu) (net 21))
 (segment (start 137.795 113.92) (end 137.795 124.0425) (width 0.6) (layer B.Cu) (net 21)))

